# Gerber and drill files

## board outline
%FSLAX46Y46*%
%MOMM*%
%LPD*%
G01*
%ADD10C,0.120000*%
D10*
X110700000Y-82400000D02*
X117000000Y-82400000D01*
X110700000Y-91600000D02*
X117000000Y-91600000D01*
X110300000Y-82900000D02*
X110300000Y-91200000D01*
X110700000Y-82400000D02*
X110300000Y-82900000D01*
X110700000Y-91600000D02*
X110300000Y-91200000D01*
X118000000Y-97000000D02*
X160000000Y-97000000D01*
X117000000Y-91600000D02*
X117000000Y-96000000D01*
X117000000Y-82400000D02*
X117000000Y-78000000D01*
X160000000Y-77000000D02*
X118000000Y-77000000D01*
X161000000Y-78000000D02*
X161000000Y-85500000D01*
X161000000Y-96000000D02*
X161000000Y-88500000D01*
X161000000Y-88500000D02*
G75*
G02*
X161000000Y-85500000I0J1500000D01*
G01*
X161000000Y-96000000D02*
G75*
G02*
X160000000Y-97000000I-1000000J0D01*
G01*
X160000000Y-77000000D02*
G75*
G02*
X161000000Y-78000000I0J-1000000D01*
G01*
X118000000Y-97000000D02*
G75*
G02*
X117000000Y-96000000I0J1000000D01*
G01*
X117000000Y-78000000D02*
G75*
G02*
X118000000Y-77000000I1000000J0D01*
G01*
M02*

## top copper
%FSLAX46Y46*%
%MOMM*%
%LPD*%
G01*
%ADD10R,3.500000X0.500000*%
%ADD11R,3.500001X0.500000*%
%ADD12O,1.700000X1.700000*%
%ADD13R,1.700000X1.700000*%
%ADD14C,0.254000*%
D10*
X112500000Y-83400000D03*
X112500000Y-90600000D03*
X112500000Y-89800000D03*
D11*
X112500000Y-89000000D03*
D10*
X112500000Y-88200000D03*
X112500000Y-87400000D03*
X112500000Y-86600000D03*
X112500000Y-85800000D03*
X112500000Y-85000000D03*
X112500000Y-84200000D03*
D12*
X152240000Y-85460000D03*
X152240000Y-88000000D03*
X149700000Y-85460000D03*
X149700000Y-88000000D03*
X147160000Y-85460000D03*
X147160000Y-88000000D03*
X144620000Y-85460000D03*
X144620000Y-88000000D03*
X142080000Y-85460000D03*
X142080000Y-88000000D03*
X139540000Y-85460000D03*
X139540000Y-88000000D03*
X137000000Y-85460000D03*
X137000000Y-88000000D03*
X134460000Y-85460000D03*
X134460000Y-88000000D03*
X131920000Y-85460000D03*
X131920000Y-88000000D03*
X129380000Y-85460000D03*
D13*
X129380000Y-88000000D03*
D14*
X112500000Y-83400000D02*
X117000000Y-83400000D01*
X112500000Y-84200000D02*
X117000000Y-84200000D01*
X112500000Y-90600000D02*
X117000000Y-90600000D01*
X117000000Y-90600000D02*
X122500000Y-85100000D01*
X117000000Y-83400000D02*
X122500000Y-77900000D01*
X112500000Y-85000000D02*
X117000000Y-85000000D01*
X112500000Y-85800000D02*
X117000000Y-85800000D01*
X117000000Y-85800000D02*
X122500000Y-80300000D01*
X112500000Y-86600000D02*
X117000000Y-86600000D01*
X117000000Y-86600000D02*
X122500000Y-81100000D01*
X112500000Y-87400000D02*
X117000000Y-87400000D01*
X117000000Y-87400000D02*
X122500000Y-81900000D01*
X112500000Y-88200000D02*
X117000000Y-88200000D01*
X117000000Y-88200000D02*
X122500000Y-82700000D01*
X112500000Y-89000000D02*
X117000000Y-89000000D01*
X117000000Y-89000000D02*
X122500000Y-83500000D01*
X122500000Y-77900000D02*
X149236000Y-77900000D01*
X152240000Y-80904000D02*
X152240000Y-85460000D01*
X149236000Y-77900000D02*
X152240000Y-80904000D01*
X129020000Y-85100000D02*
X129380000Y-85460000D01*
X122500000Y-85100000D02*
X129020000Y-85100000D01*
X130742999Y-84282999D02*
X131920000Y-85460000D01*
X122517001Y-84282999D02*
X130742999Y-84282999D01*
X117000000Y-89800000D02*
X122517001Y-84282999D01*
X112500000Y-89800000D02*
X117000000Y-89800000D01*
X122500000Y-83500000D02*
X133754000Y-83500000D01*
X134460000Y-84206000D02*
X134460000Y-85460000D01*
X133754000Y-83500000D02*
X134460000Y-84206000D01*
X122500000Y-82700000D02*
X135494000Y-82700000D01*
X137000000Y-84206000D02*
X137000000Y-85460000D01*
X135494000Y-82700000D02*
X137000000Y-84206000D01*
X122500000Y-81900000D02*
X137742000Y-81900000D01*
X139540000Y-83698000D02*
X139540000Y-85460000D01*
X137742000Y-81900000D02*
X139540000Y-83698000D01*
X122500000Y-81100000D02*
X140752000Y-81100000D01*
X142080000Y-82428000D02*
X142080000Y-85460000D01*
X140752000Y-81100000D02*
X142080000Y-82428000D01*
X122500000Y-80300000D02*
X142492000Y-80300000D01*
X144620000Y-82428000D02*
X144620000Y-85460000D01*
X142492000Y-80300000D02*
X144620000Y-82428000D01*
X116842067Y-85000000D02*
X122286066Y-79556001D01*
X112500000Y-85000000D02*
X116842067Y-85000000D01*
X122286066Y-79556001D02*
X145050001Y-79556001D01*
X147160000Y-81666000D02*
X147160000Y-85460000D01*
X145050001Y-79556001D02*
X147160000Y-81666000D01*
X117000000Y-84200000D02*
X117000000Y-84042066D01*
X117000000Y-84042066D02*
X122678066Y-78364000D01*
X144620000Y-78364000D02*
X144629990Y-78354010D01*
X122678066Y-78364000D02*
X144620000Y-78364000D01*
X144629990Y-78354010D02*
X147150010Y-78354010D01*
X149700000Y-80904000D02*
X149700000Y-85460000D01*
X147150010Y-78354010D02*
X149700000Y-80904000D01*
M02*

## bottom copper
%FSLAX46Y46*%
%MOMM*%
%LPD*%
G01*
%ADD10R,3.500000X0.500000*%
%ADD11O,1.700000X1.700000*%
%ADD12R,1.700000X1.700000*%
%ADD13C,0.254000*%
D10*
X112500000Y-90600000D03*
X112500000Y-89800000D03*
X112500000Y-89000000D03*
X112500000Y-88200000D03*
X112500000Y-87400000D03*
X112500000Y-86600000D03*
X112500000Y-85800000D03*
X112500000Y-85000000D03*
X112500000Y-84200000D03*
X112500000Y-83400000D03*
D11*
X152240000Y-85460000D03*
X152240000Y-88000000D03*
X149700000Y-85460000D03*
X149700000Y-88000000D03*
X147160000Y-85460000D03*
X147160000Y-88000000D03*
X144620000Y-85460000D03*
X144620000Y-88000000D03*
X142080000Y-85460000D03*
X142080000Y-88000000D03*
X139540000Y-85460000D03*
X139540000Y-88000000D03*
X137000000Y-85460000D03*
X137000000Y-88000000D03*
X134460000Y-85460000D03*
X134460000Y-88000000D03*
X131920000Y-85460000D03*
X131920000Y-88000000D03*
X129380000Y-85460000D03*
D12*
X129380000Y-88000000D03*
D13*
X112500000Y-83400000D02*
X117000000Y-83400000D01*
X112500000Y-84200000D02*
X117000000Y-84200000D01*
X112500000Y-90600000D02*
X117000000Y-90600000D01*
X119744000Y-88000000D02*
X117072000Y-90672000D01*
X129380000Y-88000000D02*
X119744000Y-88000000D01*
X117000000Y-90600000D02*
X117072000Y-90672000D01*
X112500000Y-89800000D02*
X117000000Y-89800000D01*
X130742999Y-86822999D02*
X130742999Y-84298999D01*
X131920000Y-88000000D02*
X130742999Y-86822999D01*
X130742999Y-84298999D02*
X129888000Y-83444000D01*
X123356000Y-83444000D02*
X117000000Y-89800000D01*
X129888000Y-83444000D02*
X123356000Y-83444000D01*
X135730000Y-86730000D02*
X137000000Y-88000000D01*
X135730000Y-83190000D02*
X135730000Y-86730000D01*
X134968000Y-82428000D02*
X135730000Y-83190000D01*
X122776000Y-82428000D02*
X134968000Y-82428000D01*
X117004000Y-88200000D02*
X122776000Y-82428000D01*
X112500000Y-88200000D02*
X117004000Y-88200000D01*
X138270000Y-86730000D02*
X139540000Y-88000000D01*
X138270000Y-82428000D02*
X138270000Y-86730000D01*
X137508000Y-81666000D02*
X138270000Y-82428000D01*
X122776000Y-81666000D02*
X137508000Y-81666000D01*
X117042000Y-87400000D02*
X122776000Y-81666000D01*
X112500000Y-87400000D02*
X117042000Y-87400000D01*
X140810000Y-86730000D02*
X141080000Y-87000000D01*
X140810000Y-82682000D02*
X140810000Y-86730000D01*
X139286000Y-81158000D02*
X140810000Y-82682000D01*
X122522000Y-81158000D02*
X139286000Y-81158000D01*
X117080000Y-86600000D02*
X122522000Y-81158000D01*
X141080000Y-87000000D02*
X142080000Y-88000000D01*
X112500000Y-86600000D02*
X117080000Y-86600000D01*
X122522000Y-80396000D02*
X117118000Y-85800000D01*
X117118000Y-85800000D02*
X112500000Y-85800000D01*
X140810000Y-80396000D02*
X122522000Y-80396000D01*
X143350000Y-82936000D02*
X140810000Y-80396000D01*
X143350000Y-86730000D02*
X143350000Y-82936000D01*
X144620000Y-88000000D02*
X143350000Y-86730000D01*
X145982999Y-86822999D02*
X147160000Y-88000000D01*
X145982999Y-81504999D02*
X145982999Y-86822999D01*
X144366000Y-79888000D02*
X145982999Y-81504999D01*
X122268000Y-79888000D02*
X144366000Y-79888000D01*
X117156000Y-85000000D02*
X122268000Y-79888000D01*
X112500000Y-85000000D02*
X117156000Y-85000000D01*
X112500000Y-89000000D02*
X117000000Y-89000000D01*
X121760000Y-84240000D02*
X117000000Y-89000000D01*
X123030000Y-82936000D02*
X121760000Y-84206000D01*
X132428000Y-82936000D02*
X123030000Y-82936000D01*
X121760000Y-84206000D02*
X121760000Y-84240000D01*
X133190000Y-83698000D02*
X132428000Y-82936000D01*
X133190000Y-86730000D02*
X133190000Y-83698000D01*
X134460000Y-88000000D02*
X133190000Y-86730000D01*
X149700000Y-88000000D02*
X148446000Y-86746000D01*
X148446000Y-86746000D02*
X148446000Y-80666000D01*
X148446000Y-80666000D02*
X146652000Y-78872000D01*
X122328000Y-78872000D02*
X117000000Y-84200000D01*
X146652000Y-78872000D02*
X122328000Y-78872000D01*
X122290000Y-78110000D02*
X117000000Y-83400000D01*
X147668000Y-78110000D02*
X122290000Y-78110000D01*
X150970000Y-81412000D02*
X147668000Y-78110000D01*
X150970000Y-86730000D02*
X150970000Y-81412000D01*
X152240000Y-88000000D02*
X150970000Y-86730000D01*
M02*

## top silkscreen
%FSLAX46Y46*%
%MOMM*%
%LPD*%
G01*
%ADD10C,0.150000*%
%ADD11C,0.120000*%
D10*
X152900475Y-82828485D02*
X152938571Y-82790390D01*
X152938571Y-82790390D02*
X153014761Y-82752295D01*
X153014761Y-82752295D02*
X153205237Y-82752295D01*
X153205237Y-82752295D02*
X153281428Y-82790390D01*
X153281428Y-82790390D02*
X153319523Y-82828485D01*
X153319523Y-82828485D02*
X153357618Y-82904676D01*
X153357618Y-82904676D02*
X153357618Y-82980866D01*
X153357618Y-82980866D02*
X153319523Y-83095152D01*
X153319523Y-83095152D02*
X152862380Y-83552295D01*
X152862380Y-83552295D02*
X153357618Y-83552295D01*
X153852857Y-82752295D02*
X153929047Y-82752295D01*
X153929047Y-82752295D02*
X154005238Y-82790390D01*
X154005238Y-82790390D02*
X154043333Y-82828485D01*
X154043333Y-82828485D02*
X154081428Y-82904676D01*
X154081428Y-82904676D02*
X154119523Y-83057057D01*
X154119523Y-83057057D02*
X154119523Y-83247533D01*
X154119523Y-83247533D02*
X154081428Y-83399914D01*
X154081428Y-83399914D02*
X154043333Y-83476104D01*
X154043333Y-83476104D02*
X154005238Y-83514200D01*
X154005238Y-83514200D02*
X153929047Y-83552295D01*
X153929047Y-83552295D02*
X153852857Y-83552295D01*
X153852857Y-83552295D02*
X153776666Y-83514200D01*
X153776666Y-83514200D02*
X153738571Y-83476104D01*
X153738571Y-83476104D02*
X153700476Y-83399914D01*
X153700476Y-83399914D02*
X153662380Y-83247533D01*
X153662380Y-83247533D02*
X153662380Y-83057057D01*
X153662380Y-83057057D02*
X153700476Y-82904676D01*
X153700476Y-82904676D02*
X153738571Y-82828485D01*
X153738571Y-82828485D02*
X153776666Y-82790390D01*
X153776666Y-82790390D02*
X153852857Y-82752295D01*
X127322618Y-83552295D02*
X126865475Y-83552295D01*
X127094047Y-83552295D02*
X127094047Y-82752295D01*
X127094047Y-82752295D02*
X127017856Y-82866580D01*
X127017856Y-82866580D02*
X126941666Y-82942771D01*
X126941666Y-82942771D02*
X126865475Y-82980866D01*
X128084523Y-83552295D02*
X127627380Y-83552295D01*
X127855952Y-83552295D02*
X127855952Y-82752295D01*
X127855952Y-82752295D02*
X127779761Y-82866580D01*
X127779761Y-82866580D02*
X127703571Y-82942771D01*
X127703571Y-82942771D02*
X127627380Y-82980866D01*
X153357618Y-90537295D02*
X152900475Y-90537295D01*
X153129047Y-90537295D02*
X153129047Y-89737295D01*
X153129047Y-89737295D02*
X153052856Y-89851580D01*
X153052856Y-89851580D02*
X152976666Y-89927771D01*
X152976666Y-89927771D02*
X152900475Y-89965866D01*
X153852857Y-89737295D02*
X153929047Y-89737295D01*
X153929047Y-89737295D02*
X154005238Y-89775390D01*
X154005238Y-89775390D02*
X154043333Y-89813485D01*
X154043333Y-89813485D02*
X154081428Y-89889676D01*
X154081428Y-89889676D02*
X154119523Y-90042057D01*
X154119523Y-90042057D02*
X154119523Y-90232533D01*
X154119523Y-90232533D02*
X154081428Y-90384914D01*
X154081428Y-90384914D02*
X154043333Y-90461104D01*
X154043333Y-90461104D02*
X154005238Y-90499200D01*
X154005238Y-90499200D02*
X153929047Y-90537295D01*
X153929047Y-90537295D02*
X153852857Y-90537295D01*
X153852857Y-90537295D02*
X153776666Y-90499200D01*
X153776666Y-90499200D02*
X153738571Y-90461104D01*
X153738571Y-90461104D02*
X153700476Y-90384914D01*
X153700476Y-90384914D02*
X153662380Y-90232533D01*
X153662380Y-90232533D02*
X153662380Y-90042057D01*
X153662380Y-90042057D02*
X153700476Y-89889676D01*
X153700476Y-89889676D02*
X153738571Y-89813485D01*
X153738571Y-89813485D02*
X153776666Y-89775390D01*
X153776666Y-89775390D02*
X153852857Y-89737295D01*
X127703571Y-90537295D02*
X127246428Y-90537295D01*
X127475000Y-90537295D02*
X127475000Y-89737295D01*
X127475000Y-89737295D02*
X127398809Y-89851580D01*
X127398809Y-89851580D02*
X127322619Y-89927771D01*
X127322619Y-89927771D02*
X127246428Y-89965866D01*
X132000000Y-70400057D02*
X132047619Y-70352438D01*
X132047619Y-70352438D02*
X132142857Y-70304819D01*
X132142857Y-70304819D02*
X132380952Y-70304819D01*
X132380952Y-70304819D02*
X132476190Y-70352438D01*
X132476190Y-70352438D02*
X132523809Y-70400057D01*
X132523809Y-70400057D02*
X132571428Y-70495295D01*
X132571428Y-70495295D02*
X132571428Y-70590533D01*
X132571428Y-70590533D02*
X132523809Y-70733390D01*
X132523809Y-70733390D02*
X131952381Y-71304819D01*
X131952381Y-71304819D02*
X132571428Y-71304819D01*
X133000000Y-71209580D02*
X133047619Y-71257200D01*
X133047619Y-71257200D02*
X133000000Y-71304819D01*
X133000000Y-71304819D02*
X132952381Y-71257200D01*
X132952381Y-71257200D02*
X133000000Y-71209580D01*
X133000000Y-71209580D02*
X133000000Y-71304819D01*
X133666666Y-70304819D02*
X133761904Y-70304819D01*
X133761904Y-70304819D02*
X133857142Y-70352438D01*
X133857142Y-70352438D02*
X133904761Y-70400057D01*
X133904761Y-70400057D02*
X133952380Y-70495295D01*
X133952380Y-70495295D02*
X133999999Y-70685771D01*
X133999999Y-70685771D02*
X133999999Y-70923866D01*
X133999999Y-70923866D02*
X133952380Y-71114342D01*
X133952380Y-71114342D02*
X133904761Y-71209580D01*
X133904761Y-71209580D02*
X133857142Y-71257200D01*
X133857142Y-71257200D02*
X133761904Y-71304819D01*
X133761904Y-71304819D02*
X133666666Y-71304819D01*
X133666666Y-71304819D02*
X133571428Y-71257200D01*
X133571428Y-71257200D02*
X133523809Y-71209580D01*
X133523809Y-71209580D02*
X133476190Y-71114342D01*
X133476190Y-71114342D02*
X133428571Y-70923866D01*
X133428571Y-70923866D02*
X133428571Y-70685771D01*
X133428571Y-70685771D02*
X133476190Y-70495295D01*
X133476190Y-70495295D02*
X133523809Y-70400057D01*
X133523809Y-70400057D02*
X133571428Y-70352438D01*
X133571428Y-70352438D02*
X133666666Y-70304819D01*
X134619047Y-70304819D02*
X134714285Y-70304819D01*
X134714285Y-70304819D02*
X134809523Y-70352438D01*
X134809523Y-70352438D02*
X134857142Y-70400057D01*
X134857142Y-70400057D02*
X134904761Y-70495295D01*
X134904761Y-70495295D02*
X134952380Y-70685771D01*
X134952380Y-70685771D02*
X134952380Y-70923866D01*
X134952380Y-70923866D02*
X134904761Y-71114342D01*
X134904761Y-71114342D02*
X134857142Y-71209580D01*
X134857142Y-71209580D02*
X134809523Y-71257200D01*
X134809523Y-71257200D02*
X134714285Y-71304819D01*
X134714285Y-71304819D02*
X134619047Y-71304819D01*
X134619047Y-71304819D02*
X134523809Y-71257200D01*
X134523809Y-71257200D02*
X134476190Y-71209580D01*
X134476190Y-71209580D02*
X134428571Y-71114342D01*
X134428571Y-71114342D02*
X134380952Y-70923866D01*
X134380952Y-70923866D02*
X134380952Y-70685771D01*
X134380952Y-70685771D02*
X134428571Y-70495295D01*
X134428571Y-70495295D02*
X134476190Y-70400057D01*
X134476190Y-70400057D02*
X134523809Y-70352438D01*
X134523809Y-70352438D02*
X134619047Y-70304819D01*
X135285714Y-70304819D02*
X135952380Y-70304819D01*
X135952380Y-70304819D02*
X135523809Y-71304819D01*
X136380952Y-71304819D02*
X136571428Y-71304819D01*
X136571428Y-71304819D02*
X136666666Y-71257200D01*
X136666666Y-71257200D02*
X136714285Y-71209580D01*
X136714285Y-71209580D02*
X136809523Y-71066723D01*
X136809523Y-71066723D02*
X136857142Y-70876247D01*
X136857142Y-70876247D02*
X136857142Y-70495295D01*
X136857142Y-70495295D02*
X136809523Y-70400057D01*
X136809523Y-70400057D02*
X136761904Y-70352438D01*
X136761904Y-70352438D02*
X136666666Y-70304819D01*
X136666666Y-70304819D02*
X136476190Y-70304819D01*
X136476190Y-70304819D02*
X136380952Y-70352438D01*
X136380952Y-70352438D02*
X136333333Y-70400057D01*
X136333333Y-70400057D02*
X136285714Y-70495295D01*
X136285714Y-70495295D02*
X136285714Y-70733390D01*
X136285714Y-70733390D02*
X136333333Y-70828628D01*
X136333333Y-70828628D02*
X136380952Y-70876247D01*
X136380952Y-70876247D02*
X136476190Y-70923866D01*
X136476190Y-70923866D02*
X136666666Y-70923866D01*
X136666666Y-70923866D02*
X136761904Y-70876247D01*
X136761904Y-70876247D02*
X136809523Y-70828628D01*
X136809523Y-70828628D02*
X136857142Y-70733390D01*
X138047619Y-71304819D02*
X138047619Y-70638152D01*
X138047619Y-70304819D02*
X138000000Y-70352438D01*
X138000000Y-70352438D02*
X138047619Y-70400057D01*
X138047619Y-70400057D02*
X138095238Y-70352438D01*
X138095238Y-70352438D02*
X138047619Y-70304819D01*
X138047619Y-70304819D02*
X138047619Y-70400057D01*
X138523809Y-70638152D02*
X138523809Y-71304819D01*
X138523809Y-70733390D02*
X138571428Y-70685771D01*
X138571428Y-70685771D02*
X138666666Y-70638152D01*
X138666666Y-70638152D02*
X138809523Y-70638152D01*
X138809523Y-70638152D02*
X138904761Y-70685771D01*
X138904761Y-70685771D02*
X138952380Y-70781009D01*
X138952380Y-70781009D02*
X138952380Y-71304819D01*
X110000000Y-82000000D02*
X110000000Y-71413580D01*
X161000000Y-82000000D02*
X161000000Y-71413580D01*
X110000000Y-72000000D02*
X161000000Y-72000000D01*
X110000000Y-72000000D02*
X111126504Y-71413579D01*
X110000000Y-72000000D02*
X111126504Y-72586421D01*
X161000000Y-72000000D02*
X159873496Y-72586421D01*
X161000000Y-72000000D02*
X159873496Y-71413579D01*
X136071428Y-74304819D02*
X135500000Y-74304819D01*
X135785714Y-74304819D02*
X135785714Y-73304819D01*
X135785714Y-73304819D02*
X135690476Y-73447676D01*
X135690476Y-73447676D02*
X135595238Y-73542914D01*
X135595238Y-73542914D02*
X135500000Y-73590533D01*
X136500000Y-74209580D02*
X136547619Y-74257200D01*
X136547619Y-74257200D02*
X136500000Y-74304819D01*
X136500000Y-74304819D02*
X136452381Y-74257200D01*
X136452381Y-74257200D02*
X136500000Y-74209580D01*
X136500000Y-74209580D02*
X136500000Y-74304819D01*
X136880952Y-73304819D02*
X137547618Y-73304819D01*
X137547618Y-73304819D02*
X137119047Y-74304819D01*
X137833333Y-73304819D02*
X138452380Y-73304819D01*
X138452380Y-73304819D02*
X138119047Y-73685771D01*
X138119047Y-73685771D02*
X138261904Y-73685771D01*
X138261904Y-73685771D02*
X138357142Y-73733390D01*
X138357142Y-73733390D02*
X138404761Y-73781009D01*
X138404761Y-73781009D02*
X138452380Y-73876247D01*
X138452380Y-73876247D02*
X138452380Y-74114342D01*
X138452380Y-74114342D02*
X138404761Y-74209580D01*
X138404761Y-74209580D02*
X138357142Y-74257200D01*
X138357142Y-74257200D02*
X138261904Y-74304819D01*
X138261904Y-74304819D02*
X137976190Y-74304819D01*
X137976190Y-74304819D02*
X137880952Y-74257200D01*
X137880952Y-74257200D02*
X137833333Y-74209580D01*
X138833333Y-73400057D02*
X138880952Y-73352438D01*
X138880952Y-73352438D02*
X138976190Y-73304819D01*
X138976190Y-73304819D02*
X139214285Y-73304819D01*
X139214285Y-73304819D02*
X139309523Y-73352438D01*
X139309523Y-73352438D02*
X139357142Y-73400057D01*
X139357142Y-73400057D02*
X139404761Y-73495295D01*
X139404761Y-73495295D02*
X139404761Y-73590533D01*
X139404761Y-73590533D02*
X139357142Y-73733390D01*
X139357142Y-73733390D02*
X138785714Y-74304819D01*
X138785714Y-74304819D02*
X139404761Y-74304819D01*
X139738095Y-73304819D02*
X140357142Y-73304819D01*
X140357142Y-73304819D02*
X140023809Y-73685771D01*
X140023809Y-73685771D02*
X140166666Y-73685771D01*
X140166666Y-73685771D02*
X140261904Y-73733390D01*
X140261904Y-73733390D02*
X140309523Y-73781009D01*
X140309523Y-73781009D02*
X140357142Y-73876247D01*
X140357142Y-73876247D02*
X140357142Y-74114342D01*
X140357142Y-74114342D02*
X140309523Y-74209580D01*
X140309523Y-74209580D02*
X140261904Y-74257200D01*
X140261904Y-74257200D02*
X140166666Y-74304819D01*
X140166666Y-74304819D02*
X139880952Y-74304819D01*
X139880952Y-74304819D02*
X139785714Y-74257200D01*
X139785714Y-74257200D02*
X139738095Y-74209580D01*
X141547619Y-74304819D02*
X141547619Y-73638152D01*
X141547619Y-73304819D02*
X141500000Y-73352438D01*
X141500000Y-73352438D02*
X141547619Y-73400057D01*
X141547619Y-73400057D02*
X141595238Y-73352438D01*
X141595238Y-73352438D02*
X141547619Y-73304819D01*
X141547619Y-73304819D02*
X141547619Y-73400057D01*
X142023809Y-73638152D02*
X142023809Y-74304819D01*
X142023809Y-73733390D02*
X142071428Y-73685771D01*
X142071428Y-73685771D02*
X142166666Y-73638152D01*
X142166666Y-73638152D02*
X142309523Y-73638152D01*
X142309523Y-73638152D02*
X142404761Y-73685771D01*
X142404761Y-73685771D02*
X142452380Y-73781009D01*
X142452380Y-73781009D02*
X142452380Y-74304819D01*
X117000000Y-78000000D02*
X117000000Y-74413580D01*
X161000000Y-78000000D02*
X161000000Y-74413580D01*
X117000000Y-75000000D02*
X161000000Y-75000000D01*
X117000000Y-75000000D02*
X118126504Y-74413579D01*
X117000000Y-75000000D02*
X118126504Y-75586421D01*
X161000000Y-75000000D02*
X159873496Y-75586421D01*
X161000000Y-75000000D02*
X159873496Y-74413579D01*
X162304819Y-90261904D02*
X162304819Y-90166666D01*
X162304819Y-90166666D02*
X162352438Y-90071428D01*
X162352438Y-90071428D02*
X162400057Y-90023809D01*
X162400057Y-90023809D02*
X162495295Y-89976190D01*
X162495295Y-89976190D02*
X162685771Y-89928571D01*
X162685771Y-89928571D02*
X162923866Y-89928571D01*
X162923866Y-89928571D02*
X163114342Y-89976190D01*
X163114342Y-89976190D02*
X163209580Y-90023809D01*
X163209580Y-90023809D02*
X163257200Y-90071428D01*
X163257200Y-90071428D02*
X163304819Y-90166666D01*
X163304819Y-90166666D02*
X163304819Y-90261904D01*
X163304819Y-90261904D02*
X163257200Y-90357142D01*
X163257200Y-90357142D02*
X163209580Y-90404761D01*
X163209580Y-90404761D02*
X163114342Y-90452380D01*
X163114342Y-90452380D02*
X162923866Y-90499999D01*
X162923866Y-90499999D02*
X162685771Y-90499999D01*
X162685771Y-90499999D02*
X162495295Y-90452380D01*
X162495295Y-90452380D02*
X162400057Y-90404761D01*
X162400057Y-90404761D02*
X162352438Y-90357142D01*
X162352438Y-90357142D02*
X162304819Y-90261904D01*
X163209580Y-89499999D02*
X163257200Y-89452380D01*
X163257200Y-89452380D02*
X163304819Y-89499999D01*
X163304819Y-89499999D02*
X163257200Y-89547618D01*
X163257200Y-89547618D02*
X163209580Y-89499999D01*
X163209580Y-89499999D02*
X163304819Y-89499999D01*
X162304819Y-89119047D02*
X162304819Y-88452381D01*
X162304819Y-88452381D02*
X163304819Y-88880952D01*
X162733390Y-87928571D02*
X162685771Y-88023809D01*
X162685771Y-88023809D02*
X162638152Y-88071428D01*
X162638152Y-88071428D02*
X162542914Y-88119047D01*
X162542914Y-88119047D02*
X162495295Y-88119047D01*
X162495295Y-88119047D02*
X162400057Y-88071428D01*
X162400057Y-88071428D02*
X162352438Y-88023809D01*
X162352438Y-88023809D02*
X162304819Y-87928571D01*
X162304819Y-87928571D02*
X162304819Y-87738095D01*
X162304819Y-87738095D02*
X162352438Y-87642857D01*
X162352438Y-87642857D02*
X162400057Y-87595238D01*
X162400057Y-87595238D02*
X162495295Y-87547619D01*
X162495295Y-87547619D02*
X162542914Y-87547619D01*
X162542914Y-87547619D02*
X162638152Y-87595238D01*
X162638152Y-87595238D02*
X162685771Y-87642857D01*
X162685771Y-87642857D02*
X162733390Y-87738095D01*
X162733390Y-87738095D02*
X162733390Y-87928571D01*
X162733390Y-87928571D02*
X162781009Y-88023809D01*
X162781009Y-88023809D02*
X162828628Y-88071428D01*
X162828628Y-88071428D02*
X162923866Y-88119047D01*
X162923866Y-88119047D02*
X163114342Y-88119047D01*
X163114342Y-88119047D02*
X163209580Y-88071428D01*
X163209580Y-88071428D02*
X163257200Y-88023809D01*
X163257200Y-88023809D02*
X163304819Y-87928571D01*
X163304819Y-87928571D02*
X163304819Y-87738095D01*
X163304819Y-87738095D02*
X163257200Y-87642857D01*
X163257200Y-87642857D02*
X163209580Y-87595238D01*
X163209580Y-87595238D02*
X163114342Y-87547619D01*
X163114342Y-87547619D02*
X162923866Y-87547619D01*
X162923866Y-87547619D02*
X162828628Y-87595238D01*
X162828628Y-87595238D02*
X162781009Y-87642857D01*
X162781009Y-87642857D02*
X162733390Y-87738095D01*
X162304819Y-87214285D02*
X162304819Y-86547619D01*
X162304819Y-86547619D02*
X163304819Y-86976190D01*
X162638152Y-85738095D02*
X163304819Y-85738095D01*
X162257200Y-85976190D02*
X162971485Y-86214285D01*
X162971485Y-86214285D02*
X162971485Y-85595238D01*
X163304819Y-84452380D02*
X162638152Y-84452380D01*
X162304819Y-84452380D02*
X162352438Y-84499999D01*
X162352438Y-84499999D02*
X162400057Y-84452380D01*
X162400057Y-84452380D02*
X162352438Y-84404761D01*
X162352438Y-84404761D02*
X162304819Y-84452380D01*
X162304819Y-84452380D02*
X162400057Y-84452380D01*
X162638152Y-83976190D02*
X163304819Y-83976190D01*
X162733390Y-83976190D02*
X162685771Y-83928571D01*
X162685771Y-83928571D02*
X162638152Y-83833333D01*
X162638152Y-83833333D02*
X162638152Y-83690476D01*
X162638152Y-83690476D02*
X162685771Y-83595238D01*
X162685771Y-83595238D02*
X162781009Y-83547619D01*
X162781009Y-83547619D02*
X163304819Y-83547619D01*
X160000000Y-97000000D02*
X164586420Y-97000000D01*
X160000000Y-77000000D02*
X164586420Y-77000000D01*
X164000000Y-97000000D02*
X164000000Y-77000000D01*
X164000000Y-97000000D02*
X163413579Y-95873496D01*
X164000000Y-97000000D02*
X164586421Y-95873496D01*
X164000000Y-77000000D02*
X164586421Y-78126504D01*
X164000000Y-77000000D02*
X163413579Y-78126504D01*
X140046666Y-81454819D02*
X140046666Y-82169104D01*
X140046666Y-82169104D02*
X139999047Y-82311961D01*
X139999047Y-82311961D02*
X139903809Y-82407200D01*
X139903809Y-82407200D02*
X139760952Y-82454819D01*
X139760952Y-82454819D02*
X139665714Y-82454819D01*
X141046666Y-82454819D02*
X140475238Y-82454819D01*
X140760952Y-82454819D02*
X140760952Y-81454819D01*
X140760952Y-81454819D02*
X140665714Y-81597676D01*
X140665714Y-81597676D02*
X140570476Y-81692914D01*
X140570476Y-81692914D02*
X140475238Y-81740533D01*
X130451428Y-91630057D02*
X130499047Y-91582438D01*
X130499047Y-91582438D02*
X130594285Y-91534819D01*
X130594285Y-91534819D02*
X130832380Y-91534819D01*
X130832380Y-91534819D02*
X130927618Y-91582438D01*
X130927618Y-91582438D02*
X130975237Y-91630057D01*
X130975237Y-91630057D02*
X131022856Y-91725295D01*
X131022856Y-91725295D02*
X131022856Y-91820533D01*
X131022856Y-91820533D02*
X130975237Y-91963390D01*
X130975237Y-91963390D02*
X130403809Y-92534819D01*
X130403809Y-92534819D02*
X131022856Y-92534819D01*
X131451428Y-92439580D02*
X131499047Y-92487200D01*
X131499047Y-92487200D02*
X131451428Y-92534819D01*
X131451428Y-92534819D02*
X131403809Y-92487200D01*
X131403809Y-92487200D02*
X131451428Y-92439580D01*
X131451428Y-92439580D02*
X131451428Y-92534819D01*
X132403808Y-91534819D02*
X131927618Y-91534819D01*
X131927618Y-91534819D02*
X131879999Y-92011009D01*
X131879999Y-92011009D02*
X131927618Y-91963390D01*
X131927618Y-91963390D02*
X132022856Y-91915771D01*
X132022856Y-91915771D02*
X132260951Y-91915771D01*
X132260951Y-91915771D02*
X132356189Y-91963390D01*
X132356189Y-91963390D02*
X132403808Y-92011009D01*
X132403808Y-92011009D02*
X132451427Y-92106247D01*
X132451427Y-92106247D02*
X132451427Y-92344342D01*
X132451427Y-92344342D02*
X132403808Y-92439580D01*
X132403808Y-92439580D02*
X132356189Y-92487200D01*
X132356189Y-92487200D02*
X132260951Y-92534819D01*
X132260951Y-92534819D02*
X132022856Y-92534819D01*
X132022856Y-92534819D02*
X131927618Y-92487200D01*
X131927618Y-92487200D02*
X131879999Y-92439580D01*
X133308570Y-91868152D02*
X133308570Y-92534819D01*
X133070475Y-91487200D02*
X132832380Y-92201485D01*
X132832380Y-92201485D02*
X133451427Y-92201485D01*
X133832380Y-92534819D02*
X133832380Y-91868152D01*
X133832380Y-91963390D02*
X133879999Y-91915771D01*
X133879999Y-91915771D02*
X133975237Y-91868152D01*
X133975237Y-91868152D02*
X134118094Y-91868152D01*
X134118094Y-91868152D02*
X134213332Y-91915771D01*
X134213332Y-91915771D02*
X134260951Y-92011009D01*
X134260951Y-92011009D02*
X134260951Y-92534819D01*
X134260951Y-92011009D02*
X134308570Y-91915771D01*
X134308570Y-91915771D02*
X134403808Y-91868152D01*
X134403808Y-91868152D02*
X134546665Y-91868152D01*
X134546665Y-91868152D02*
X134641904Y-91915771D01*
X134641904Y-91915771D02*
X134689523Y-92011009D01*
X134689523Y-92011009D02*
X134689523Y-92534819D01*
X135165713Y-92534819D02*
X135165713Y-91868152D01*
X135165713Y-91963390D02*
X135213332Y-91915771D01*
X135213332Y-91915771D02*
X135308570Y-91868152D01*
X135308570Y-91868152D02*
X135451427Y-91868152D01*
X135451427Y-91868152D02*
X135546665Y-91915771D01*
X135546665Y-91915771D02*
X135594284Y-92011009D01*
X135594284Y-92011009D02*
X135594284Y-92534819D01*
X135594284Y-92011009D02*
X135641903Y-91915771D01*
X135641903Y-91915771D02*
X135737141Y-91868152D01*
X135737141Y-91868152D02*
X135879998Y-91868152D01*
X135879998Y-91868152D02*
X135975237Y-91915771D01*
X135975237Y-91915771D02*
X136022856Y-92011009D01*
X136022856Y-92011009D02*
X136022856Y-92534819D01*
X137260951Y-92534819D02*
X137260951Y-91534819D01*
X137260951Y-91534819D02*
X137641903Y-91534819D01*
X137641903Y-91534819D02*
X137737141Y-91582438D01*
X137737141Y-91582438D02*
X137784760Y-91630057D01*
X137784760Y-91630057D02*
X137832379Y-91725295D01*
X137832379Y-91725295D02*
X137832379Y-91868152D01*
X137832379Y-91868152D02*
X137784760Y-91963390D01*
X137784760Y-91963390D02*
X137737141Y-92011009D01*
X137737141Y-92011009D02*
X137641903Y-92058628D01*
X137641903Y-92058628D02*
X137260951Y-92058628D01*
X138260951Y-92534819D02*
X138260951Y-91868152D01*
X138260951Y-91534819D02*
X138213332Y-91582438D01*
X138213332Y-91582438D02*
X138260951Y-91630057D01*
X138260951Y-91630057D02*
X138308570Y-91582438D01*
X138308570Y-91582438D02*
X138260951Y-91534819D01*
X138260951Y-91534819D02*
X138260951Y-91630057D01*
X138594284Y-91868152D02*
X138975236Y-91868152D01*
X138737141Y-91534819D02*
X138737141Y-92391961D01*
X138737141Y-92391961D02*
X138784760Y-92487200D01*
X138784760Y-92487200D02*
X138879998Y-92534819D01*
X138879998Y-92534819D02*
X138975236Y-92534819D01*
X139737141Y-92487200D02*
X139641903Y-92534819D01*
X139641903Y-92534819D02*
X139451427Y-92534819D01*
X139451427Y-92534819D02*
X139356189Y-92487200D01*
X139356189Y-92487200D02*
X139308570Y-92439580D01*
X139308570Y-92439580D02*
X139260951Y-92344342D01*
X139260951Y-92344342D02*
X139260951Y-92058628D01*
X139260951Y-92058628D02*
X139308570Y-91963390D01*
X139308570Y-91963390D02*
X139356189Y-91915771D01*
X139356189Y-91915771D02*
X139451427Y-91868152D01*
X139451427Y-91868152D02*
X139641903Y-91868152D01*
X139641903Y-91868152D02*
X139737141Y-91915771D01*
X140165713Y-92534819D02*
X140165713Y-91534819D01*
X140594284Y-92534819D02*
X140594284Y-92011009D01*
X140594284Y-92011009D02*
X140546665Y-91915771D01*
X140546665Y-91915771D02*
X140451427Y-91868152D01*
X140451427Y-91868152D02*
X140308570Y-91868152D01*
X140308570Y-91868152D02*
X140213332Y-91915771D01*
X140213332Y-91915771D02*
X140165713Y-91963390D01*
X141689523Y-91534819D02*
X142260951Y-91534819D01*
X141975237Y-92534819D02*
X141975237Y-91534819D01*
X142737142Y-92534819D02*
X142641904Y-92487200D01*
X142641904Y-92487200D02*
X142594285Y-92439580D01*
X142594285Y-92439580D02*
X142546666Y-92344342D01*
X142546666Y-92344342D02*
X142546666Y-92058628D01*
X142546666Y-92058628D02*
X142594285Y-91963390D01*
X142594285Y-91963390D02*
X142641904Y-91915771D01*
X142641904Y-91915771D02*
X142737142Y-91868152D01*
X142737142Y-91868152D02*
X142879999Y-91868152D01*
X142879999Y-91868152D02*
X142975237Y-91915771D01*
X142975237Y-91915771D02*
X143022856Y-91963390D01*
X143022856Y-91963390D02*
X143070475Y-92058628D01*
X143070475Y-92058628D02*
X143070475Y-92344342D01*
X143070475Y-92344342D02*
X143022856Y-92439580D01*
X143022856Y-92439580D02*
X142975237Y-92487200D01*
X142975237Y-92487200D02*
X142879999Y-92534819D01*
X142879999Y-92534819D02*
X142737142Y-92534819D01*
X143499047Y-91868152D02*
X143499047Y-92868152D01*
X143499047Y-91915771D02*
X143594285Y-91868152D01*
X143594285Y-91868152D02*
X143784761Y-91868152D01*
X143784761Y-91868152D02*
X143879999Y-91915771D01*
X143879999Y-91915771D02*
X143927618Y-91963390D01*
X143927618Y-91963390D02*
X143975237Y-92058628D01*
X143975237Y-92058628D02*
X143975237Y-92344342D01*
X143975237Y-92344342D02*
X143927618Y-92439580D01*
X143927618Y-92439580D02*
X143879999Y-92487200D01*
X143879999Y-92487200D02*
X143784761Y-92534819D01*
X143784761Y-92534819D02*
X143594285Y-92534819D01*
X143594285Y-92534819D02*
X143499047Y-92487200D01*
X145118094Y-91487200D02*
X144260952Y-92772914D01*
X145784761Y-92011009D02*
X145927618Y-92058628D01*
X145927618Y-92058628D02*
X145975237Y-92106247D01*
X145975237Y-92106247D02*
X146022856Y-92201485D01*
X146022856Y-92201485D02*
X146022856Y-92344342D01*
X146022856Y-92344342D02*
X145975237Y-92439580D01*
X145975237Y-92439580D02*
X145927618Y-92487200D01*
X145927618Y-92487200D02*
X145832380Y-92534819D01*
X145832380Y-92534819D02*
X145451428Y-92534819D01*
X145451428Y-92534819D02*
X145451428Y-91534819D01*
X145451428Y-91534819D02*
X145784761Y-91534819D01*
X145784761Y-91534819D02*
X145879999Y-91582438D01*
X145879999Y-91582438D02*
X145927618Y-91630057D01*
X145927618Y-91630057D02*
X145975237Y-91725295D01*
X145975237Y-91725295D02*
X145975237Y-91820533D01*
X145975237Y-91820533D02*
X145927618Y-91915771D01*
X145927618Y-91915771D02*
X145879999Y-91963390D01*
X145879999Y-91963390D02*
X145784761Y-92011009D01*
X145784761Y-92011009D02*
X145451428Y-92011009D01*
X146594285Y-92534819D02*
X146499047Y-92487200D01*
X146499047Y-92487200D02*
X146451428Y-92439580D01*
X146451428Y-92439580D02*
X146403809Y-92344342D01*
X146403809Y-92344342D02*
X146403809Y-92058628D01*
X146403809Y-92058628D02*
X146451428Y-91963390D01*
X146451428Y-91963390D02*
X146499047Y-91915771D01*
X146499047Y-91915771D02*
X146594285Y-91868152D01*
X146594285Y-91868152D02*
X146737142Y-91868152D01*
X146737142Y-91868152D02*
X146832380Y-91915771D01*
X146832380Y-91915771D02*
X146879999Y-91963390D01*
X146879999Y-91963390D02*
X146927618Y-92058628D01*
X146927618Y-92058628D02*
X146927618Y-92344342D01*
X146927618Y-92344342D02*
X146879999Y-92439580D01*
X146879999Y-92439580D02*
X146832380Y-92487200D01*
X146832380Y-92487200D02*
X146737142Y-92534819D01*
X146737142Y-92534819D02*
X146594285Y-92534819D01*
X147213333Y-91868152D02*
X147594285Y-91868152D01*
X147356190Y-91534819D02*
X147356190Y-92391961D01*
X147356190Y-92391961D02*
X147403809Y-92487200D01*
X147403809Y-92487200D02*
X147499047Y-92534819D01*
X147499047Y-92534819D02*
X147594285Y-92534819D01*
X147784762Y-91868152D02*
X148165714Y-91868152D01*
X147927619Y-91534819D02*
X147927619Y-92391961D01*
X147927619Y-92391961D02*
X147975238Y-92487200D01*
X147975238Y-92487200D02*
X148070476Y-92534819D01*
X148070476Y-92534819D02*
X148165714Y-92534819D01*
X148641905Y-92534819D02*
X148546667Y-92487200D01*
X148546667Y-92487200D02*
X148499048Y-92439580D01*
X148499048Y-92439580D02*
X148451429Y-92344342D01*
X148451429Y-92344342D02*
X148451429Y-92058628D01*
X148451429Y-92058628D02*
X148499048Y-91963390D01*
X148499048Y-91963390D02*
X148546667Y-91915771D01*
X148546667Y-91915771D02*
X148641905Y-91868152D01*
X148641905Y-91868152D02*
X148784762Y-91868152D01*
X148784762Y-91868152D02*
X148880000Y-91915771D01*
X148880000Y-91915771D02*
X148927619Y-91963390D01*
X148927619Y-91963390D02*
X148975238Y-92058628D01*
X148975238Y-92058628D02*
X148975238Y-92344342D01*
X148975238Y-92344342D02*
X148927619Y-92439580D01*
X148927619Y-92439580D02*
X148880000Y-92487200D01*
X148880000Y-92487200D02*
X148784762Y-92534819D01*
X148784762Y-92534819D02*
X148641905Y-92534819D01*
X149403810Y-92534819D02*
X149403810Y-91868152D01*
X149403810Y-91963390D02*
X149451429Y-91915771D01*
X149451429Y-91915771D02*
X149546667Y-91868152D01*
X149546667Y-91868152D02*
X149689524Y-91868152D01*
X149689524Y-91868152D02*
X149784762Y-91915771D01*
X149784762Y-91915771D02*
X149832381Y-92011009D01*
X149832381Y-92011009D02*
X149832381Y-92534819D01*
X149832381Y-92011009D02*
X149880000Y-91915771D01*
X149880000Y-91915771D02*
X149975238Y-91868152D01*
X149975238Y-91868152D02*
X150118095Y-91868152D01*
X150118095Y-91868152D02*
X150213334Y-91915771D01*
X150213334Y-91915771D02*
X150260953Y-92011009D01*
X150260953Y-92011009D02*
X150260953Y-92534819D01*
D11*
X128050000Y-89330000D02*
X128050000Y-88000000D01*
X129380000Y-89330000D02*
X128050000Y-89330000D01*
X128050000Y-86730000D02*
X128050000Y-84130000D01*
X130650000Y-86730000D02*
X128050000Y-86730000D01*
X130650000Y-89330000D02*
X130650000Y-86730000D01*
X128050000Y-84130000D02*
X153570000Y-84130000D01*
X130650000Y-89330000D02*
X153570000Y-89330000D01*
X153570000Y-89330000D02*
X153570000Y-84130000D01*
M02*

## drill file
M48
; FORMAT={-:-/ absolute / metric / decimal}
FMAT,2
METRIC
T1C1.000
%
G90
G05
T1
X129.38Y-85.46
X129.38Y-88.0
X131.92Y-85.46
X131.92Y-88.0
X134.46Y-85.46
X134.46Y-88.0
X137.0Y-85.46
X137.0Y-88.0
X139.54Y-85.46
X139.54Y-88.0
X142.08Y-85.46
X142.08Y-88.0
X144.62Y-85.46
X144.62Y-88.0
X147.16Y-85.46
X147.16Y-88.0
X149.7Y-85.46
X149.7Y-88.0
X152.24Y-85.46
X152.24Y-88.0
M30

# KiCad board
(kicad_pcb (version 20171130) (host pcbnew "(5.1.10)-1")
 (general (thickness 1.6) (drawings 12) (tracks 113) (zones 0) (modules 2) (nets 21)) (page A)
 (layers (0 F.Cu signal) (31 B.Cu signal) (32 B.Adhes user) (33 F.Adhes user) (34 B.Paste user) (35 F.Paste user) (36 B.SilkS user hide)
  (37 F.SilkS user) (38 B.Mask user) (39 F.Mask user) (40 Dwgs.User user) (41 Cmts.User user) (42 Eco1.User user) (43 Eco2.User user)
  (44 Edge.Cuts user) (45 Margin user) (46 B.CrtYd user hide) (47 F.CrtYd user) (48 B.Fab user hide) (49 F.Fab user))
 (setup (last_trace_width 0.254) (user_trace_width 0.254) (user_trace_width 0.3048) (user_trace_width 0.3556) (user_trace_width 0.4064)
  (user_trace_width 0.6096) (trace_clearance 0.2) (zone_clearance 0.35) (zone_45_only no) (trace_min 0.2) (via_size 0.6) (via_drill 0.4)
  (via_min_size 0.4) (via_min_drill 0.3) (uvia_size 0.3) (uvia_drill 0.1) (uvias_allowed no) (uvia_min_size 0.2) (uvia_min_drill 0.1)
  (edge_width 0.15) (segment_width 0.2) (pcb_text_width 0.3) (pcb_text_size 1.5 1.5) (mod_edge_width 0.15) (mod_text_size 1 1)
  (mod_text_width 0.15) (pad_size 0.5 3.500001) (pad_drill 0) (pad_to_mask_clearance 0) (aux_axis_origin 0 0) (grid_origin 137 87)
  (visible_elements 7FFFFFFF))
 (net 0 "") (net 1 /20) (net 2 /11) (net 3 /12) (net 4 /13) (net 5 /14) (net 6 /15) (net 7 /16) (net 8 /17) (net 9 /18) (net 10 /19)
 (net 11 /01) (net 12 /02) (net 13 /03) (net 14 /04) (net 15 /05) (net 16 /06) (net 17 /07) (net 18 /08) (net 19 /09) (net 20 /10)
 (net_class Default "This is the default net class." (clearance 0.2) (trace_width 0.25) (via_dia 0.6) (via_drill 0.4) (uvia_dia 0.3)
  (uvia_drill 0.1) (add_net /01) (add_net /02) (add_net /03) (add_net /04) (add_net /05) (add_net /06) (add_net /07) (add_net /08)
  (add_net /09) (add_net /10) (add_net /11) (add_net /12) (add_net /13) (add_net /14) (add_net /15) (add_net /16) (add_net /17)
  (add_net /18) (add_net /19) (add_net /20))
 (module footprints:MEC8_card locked (layer F.Cu) (at 112.5 87 90)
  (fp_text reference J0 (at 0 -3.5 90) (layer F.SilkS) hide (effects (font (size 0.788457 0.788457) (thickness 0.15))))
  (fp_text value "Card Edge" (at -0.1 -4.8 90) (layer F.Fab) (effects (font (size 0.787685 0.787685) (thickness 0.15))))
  (fp_line (start 4.6 -1.8) (end 4.6 4.5) (layer Edge.Cuts) (width 0.12))
  (fp_line (start -4.6 -1.8) (end -4.6 4.5) (layer Edge.Cuts) (width 0.12))
  (fp_line (start 4.1 -2.2) (end -4.2 -2.2) (layer Edge.Cuts) (width 0.12))
  (fp_line (start 4.6 -1.8) (end 4.1 -2.2) (layer Edge.Cuts) (width 0.12))
  (fp_line (start -4.6 -1.8) (end -4.2 -2.2) (layer Edge.Cuts) (width 0.12))
  (fp_line (start -10 5.5) (end -10 47.5) (layer Edge.Cuts) (width 0.12))
  (fp_line (start -4.6 4.5) (end -9 4.5) (layer Edge.Cuts) (width 0.12))
  (fp_line (start 4.6 4.5) (end 9 4.5) (layer Edge.Cuts) (width 0.12))
  (fp_line (start 10 47.5) (end 10 5.5) (layer Edge.Cuts) (width 0.12))
  (fp_line (start 9 48.5) (end 1.5 48.5) (layer Edge.Cuts) (width 0.12))
  (fp_line (start -9 48.5) (end -1.5 48.5) (layer Edge.Cuts) (width 0.12))
  (fp_arc (start 0 48.5) (end 1.5 48.5) (angle -180) (layer Edge.Cuts) (width 0.12))
  (fp_arc (start -9 47.5) (end -10 47.5) (angle -90) (layer Edge.Cuts) (width 0.12))
  (fp_arc (start 9 47.5) (end 9 48.5) (angle -90) (layer Edge.Cuts) (width 0.12))
  (fp_arc (start -9 5.5) (end -9 4.5) (angle -90) (layer Edge.Cuts) (width 0.12))
  (fp_arc (start 9 5.5) (end 10 5.5) (angle -90) (layer Edge.Cuts) (width 0.12))
  (pad 20 smd rect (at 3.6 0 90) (size 0.5 3.5) (layers F.Cu F.Paste F.Mask) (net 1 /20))
  (pad 11 smd rect (at -3.6 0 90) (size 0.5 3.5) (layers F.Cu F.Paste F.Mask) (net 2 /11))
  (pad 12 smd rect (at -2.8 0 90) (size 0.5 3.5) (layers F.Cu F.Paste F.Mask) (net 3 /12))
  (pad 13 smd rect (at -2 0 90) (size 0.5 3.500001) (layers F.Cu F.Paste F.Mask) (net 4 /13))
  (pad 14 smd rect (at -1.2 0 90) (size 0.5 3.5) (layers F.Cu F.Paste F.Mask) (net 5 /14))
  (pad 15 smd rect (at -0.4 0 90) (size 0.5 3.5) (layers F.Cu F.Paste F.Mask) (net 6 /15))
  (pad 16 smd rect (at 0.4 0 90) (size 0.5 3.5) (layers F.Cu F.Paste F.Mask) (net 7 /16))
  (pad 17 smd rect (at 1.2 0 90) (size 0.5 3.5) (layers F.Cu F.Paste F.Mask) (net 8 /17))
  (pad 18 smd rect (at 2 0 90) (size 0.5 3.5) (layers F.Cu F.Paste F.Mask) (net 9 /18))
  (pad 19 smd rect (at 2.8 0 90) (size 0.5 3.5) (layers F.Cu F.Paste F.Mask) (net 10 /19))
  (pad 1 smd rect (at -3.6 0 90) (size 0.5 3.5) (layers B.Cu B.Paste B.Mask) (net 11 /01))
  (pad 2 smd rect (at -2.8 0 90) (size 0.5 3.5) (layers B.Cu B.Paste B.Mask) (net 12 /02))
  (pad 3 smd rect (at -2 0 90) (size 0.5 3.5) (layers B.Cu B.Paste B.Mask) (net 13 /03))
  (pad 4 smd rect (at -1.2 0 90) (size 0.5 3.5) (layers B.Cu B.Paste B.Mask) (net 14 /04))
  (pad 5 smd rect (at -0.4 0 90) (size 0.5 3.5) (layers B.Cu B.Paste B.Mask) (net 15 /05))
  (pad 6 smd rect (at 0.4 0 90) (size 0.5 3.5) (layers B.Cu B.Paste B.Mask) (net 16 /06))
  (pad 7 smd rect (at 1.2 0 90) (size 0.5 3.5) (layers B.Cu B.Paste B.Mask) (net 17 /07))
  (pad 8 smd rect (at 2 0 90) (size 0.5 3.5) (layers B.Cu B.Paste B.Mask) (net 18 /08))
  (pad 9 smd rect (at 2.8 0 90) (size 0.5 3.5) (layers B.Cu B.Paste B.Mask) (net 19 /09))
  (pad 10 smd rect (at 3.6 0 90) (size 0.5 3.5) (layers B.Cu B.Paste B.Mask) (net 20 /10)))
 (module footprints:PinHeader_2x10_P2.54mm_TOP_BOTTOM (layer F.Cu) (at 129.38 88 90)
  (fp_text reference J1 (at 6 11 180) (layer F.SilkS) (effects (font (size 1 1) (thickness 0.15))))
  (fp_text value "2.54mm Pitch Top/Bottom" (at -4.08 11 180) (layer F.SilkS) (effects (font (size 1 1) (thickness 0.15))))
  (fp_line (start -1.33 -1.33) (end 0 -1.33) (layer F.SilkS) (width 0.12))
  (fp_line (start -1.33 0) (end -1.33 -1.33) (layer F.SilkS) (width 0.12))
  (fp_line (start 1.27 -1.33) (end 3.87 -1.33) (layer F.SilkS) (width 0.12))
  (fp_line (start 1.27 1.27) (end 1.27 -1.33) (layer F.SilkS) (width 0.12))
  (fp_line (start -1.33 1.27) (end 1.27 1.27) (layer F.SilkS) (width 0.12))
  (fp_line (start 3.87 -1.33) (end 3.87 24.19) (layer F.SilkS) (width 0.12))
  (fp_line (start -1.33 1.27) (end -1.33 24.19) (layer F.SilkS) (width 0.12))
  (fp_line (start -1.33 24.19) (end 3.87 24.19) (layer F.SilkS) (width 0.12))
  (pad 20 thru_hole oval (at 2.54 22.86 90) (size 1.7 1.7) (drill 1) (layers *.Cu *.Mask) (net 1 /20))
  (pad 10 thru_hole oval (at 0 22.86 90) (size 1.7 1.7) (drill 1) (layers *.Cu *.Mask) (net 20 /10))
  (pad 19 thru_hole oval (at 2.54 20.32 90) (size 1.7 1.7) (drill 1) (layers *.Cu *.Mask) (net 10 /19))
  (pad 9 thru_hole oval (at 0 20.32 90) (size 1.7 1.7) (drill 1) (layers *.Cu *.Mask) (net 19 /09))
  (pad 18 thru_hole oval (at 2.54 17.78 90) (size 1.7 1.7) (drill 1) (layers *.Cu *.Mask) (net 9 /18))
  (pad 8 thru_hole oval (at 0 17.78 90) (size 1.7 1.7) (drill 1) (layers *.Cu *.Mask) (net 18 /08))
  (pad 17 thru_hole oval (at 2.54 15.24 90) (size 1.7 1.7) (drill 1) (layers *.Cu *.Mask) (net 8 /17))
  (pad 7 thru_hole oval (at 0 15.24 90) (size 1.7 1.7) (drill 1) (layers *.Cu *.Mask) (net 17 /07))
  (pad 16 thru_hole oval (at 2.54 12.7 90) (size 1.7 1.7) (drill 1) (layers *.Cu *.Mask) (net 7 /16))
  (pad 6 thru_hole oval (at 0 12.7 90) (size 1.7 1.7) (drill 1) (layers *.Cu *.Mask) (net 16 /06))
  (pad 15 thru_hole oval (at 2.54 10.16 90) (size 1.7 1.7) (drill 1) (layers *.Cu *.Mask) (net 6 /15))
  (pad 5 thru_hole oval (at 0 10.16 90) (size 1.7 1.7) (drill 1) (layers *.Cu *.Mask) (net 15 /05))
  (pad 14 thru_hole oval (at 2.54 7.62 90) (size 1.7 1.7) (drill 1) (layers *.Cu *.Mask) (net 5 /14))
  (pad 4 thru_hole oval (at 0 7.62 90) (size 1.7 1.7) (drill 1) (layers *.Cu *.Mask) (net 14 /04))
  (pad 13 thru_hole oval (at 2.54 5.08 90) (size 1.7 1.7) (drill 1) (layers *.Cu *.Mask) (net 4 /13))
  (pad 3 thru_hole oval (at 0 5.08 90) (size 1.7 1.7) (drill 1) (layers *.Cu *.Mask) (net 13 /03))
  (pad 12 thru_hole oval (at 2.54 2.54 90) (size 1.7 1.7) (drill 1) (layers *.Cu *.Mask) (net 3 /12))
  (pad 2 thru_hole oval (at 0 2.54 90) (size 1.7 1.7) (drill 1) (layers *.Cu *.Mask) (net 12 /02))
  (pad 11 thru_hole oval (at 2.54 0 90) (size 1.7 1.7) (drill 1) (layers *.Cu *.Mask) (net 2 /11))
  (pad 1 thru_hole rect (at 0 0 90) (size 1.7 1.7) (drill 1) (layers *.Cu *.Mask) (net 11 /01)))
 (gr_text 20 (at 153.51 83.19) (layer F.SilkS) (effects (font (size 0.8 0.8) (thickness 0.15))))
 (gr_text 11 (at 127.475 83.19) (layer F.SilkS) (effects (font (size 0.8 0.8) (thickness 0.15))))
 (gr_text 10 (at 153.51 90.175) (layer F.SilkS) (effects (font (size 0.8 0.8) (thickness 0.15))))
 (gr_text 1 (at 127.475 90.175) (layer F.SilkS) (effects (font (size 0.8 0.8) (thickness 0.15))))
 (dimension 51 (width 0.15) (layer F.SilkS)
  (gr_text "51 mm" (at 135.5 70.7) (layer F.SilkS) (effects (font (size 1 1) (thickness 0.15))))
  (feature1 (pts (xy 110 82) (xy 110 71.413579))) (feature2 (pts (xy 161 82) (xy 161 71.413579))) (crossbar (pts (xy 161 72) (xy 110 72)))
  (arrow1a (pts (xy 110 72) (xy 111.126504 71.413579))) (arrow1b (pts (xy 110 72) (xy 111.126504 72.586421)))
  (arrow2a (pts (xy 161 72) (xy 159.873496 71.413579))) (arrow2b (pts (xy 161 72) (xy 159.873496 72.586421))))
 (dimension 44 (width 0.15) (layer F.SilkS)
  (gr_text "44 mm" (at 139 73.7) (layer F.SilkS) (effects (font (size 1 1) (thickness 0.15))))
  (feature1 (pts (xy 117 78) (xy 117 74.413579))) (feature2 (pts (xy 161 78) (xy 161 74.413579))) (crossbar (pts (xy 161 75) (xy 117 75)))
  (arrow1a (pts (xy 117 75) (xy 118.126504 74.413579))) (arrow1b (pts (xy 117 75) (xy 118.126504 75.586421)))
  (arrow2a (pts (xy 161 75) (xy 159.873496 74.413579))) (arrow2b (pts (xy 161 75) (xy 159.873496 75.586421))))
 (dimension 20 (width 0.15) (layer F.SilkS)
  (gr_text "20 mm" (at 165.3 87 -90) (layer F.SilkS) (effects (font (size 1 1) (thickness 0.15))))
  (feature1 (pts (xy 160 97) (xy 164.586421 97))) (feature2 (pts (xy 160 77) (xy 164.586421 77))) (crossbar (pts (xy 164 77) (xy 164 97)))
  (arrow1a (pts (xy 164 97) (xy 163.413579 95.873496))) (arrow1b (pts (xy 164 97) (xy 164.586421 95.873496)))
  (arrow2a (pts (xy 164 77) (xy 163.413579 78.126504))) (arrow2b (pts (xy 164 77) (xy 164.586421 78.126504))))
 (segment (start 112.5 83.4) (end 117 83.4) (width 0.254) (layer F.Cu) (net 1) (status 10))
 (segment (start 112.5 84.2) (end 117 84.2) (width 0.254) (layer F.Cu) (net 10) (status 10))
 (segment (start 112.5 90.6) (end 117 90.6) (width 0.254) (layer F.Cu) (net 2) (status 10))
 (segment (start 117 90.6) (end 122.5 85.1) (width 0.254) (layer F.Cu) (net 2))
 (segment (start 117 83.4) (end 122.5 77.9) (width 0.254) (layer F.Cu) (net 1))
 (segment (start 112.5 83.4) (end 117 83.4) (width 0.254) (layer B.Cu) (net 20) (status 10))
 (segment (start 112.5 85) (end 117 85) (width 0.254) (layer F.Cu) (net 9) (status 10))
 (segment (start 112.5 85.8) (end 117 85.8) (width 0.254) (layer F.Cu) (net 8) (status 10))
 (segment (start 117 85.8) (end 122.5 80.3) (width 0.254) (layer F.Cu) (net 8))
 (segment (start 112.5 86.6) (end 117 86.6) (width 0.254) (layer F.Cu) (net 7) (status 10))
 (segment (start 117 86.6) (end 122.5 81.1) (width 0.254) (layer F.Cu) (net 7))
 (segment (start 112.5 87.4) (end 117 87.4) (width 0.254) (layer F.Cu) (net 6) (status 10))
 (segment (start 117 87.4) (end 122.5 81.9) (width 0.254) (layer F.Cu) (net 6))
 (segment (start 112.5 88.2) (end 117 88.2) (width 0.254) (layer F.Cu) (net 5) (status 10))
 (segment (start 117 88.2) (end 122.5 82.7) (width 0.254) (layer F.Cu) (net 5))
 (segment (start 112.5 89) (end 117 89) (width 0.254) (layer F.Cu) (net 4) (status 10))
 (segment (start 117 89) (end 122.5 83.5) (width 0.254) (layer F.Cu) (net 4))
 (segment (start 112.5 84.2) (end 117 84.2) (width 0.254) (layer B.Cu) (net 19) (status 10))
 (segment (start 112.5 90.6) (end 117 90.6) (width 0.254) (layer B.Cu) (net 11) (status 10))
 (segment (start 119.744 88) (end 117.072 90.672) (width 0.254) (layer B.Cu) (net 11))
 (segment (start 129.38 88) (end 119.744 88) (width 0.254) (layer B.Cu) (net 11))
 (segment (start 117 90.6) (end 117.072 90.672) (width 0.254) (layer B.Cu) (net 11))
 (segment (start 112.5 89.8) (end 117 89.8) (width 0.254) (layer B.Cu) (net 12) (status 10))
 (segment (start 130.742999 86.822999) (end 130.742999 84.298999) (width 0.254) (layer B.Cu) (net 12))
 (segment (start 131.92 88) (end 130.742999 86.822999) (width 0.254) (layer B.Cu) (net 12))
 (segment (start 130.742999 84.298999) (end 129.888 83.444) (width 0.254) (layer B.Cu) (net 12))
 (segment (start 123.356 83.444) (end 117 89.8) (width 0.254) (layer B.Cu) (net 12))
 (segment (start 129.888 83.444) (end 123.356 83.444) (width 0.254) (layer B.Cu) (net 12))
 (segment (start 135.73 86.73) (end 137 88) (width 0.254) (layer B.Cu) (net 14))
 (segment (start 135.73 83.19) (end 135.73 86.73) (width 0.254) (layer B.Cu) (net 14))
 (segment (start 134.968 82.428) (end 135.73 83.19) (width 0.254) (layer B.Cu) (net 14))
 (segment (start 122.776 82.428) (end 134.968 82.428) (width 0.254) (layer B.Cu) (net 14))
 (segment (start 117.004 88.2) (end 122.776 82.428) (width 0.254) (layer B.Cu) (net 14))
 (segment (start 112.5 88.2) (end 117.004 88.2) (width 0.254) (layer B.Cu) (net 14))
 (segment (start 138.27 86.73) (end 139.54 88) (width 0.254) (layer B.Cu) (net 15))
 (segment (start 138.27 82.428) (end 138.27 86.73) (width 0.254) (layer B.Cu) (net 15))
 (segment (start 137.508 81.666) (end 138.27 82.428) (width 0.254) (layer B.Cu) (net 15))
 (segment (start 122.776 81.666) (end 137.508 81.666) (width 0.254) (layer B.Cu) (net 15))
 (segment (start 117.042 87.4) (end 122.776 81.666) (width 0.254) (layer B.Cu) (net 15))
 (segment (start 112.5 87.4) (end 117.042 87.4) (width 0.254) (layer B.Cu) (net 15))
 (segment (start 140.81 86.73) (end 141.08 87) (width 0.254) (layer B.Cu) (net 16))
 (segment (start 140.81 82.682) (end 140.81 86.73) (width 0.254) (layer B.Cu) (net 16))
 (segment (start 139.286 81.158) (end 140.81 82.682) (width 0.254) (layer B.Cu) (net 16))
 (segment (start 122.522 81.158) (end 139.286 81.158) (width 0.254) (layer B.Cu) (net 16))
 (segment (start 117.08 86.6) (end 122.522 81.158) (width 0.254) (layer B.Cu) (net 16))
 (segment (start 141.08 87) (end 142.08 88) (width 0.254) (layer B.Cu) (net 16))
 (segment (start 112.5 86.6) (end 117.08 86.6) (width 0.254) (layer B.Cu) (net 16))
 (segment (start 122.522 80.396) (end 117.118 85.8) (width 0.254) (layer B.Cu) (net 17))
 (segment (start 117.118 85.8) (end 112.5 85.8) (width 0.254) (layer B.Cu) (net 17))
 (segment (start 140.81 80.396) (end 122.522 80.396) (width 0.254) (layer B.Cu) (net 17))
 (segment (start 143.35 82.936) (end 140.81 80.396) (width 0.254) (layer B.Cu) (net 17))
 (segment (start 143.35 86.73) (end 143.35 82.936) (width 0.254) (layer B.Cu) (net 17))
 (segment (start 144.62 88) (end 143.35 86.73) (width 0.254) (layer B.Cu) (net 17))
 (segment (start 145.982999 86.822999) (end 147.16 88) (width 0.254) (layer B.Cu) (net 18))
 (segment (start 145.982999 81.504999) (end 145.982999 86.822999) (width 0.254) (layer B.Cu) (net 18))
 (segment (start 144.366 79.888) (end 145.982999 81.504999) (width 0.254) (layer B.Cu) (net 18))
 (segment (start 122.268 79.888) (end 144.366 79.888) (width 0.254) (layer B.Cu) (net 18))
 (segment (start 117.156 85) (end 122.268 79.888) (width 0.254) (layer B.Cu) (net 18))
 (segment (start 112.5 85) (end 117.156 85) (width 0.254) (layer B.Cu) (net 18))
 (segment (start 112.5 89) (end 117 89) (width 0.254) (layer B.Cu) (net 13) (status 10))
 (segment (start 121.76 84.24) (end 117 89) (width 0.254) (layer B.Cu) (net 13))
 (segment (start 123.03 82.936) (end 121.76 84.206) (width 0.254) (layer B.Cu) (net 13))
 (segment (start 132.428 82.936) (end 123.03 82.936) (width 0.254) (layer B.Cu) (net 13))
 (segment (start 121.76 84.206) (end 121.76 84.24) (width 0.254) (layer B.Cu) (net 13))
 (segment (start 133.19 83.698) (end 132.428 82.936) (width 0.254) (layer B.Cu) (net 13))
 (segment (start 133.19 86.73) (end 133.19 83.698) (width 0.254) (layer B.Cu) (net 13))
 (segment (start 134.46 88) (end 133.19 86.73) (width 0.254) (layer B.Cu) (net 13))
 (segment (start 122.5 77.9) (end 149.236 77.9) (width 0.254) (layer F.Cu) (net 1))
 (segment (start 152.24 80.904) (end 152.24 85.46) (width 0.254) (layer F.Cu) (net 1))
 (segment (start 149.236 77.9) (end 152.24 80.904) (width 0.254) (layer F.Cu) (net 1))
 (segment (start 129.02 85.1) (end 129.38 85.46) (width 0.254) (layer F.Cu) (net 2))
 (segment (start 122.5 85.1) (end 129.02 85.1) (width 0.254) (layer F.Cu) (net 2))
 (segment (start 130.742999 84.282999) (end 131.92 85.46) (width 0.254) (layer F.Cu) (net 3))
 (segment (start 122.517001 84.282999) (end 130.742999 84.282999) (width 0.254) (layer F.Cu) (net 3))
 (segment (start 117 89.8) (end 122.517001 84.282999) (width 0.254) (layer F.Cu) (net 3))
 (segment (start 112.5 89.8) (end 117 89.8) (width 0.254) (layer F.Cu) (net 3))
 (segment (start 122.5 83.5) (end 133.754 83.5) (width 0.254) (layer F.Cu) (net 4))
 (segment (start 134.46 84.206) (end 134.46 85.46) (width 0.254) (layer F.Cu) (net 4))
 (segment (start 133.754 83.5) (end 134.46 84.206) (width 0.254) (layer F.Cu) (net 4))
 (segment (start 122.5 82.7) (end 135.494 82.7) (width 0.254) (layer F.Cu) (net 5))
 (segment (start 137 84.206) (end 137 85.46) (width 0.254) (layer F.Cu) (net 5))
 (segment (start 135.494 82.7) (end 137 84.206) (width 0.254) (layer F.Cu) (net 5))
 (segment (start 122.5 81.9) (end 137.742 81.9) (width 0.254) (layer F.Cu) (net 6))
 (segment (start 139.54 83.698) (end 139.54 85.46) (width 0.254) (layer F.Cu) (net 6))
 (segment (start 137.742 81.9) (end 139.54 83.698) (width 0.254) (layer F.Cu) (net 6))
 (segment (start 122.5 81.1) (end 140.752 81.1) (width 0.254) (layer F.Cu) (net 7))
 (segment (start 142.08 82.428) (end 142.08 85.46) (width 0.254) (layer F.Cu) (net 7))
 (segment (start 140.752 81.1) (end 142.08 82.428) (width 0.254) (layer F.Cu) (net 7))
 (segment (start 122.5 80.3) (end 142.492 80.3) (width 0.254) (layer F.Cu) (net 8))
 (segment (start 144.62 82.428) (end 144.62 85.46) (width 0.254) (layer F.Cu) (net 8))
 (segment (start 142.492 80.3) (end 144.62 82.428) (width 0.254) (layer F.Cu) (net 8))
 (segment (start 116.842067 85) (end 122.286066 79.556001) (width 0.254) (layer F.Cu) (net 9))
 (segment (start 112.5 85) (end 116.842067 85) (width 0.254) (layer F.Cu) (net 9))
 (segment (start 122.286066 79.556001) (end 145.050001 79.556001) (width 0.254) (layer F.Cu) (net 9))
 (segment (start 147.16 81.666) (end 147.16 85.46) (width 0.254) (layer F.Cu) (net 9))
 (segment (start 145.050001 79.556001) (end 147.16 81.666) (width 0.254) (layer F.Cu) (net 9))
 (segment (start 117 84.2) (end 117 84.042066) (width 0.254) (layer F.Cu) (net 10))
 (segment (start 117 84.042066) (end 122.678066 78.364) (width 0.254) (layer F.Cu) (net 10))
 (segment (start 144.62 78.364) (end 144.62999 78.35401) (width 0.254) (layer F.Cu) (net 10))
 (segment (start 122.678066 78.364) (end 144.62 78.364) (width 0.254) (layer F.Cu) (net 10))
 (segment (start 144.62999 78.35401) (end 147.15001 78.35401) (width 0.254) (layer F.Cu) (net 10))
 (segment (start 149.7 80.904) (end 149.7 85.46) (width 0.254) (layer F.Cu) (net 10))
 (segment (start 147.15001 78.35401) (end 149.7 80.904) (width 0.254) (layer F.Cu) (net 10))
 (segment (start 149.7 88) (end 148.446 86.746) (width 0.254) (layer B.Cu) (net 19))
 (segment (start 148.446 86.746) (end 148.446 80.666) (width 0.254) (layer B.Cu) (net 19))
 (segment (start 148.446 80.666) (end 146.652 78.872) (width 0.254) (layer B.Cu) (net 19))
 (segment (start 122.328 78.872) (end 117 84.2) (width 0.254) (layer B.Cu) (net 19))
 (segment (start 146.652 78.872) (end 122.328 78.872) (width 0.254) (layer B.Cu) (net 19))
 (segment (start 122.29 78.11) (end 117 83.4) (width 0.254) (layer B.Cu) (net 20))
 (segment (start 147.668 78.11) (end 122.29 78.11) (width 0.254) (layer B.Cu) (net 20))
 (segment (start 150.97 81.412) (end 147.668 78.11) (width 0.254) (layer B.Cu) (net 20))
 (segment (start 150.97 86.73) (end 150.97 81.412) (width 0.254) (layer B.Cu) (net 20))
 (segment (start 152.24 88) (end 150.97 86.73) (width 0.254) (layer B.Cu) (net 20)))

